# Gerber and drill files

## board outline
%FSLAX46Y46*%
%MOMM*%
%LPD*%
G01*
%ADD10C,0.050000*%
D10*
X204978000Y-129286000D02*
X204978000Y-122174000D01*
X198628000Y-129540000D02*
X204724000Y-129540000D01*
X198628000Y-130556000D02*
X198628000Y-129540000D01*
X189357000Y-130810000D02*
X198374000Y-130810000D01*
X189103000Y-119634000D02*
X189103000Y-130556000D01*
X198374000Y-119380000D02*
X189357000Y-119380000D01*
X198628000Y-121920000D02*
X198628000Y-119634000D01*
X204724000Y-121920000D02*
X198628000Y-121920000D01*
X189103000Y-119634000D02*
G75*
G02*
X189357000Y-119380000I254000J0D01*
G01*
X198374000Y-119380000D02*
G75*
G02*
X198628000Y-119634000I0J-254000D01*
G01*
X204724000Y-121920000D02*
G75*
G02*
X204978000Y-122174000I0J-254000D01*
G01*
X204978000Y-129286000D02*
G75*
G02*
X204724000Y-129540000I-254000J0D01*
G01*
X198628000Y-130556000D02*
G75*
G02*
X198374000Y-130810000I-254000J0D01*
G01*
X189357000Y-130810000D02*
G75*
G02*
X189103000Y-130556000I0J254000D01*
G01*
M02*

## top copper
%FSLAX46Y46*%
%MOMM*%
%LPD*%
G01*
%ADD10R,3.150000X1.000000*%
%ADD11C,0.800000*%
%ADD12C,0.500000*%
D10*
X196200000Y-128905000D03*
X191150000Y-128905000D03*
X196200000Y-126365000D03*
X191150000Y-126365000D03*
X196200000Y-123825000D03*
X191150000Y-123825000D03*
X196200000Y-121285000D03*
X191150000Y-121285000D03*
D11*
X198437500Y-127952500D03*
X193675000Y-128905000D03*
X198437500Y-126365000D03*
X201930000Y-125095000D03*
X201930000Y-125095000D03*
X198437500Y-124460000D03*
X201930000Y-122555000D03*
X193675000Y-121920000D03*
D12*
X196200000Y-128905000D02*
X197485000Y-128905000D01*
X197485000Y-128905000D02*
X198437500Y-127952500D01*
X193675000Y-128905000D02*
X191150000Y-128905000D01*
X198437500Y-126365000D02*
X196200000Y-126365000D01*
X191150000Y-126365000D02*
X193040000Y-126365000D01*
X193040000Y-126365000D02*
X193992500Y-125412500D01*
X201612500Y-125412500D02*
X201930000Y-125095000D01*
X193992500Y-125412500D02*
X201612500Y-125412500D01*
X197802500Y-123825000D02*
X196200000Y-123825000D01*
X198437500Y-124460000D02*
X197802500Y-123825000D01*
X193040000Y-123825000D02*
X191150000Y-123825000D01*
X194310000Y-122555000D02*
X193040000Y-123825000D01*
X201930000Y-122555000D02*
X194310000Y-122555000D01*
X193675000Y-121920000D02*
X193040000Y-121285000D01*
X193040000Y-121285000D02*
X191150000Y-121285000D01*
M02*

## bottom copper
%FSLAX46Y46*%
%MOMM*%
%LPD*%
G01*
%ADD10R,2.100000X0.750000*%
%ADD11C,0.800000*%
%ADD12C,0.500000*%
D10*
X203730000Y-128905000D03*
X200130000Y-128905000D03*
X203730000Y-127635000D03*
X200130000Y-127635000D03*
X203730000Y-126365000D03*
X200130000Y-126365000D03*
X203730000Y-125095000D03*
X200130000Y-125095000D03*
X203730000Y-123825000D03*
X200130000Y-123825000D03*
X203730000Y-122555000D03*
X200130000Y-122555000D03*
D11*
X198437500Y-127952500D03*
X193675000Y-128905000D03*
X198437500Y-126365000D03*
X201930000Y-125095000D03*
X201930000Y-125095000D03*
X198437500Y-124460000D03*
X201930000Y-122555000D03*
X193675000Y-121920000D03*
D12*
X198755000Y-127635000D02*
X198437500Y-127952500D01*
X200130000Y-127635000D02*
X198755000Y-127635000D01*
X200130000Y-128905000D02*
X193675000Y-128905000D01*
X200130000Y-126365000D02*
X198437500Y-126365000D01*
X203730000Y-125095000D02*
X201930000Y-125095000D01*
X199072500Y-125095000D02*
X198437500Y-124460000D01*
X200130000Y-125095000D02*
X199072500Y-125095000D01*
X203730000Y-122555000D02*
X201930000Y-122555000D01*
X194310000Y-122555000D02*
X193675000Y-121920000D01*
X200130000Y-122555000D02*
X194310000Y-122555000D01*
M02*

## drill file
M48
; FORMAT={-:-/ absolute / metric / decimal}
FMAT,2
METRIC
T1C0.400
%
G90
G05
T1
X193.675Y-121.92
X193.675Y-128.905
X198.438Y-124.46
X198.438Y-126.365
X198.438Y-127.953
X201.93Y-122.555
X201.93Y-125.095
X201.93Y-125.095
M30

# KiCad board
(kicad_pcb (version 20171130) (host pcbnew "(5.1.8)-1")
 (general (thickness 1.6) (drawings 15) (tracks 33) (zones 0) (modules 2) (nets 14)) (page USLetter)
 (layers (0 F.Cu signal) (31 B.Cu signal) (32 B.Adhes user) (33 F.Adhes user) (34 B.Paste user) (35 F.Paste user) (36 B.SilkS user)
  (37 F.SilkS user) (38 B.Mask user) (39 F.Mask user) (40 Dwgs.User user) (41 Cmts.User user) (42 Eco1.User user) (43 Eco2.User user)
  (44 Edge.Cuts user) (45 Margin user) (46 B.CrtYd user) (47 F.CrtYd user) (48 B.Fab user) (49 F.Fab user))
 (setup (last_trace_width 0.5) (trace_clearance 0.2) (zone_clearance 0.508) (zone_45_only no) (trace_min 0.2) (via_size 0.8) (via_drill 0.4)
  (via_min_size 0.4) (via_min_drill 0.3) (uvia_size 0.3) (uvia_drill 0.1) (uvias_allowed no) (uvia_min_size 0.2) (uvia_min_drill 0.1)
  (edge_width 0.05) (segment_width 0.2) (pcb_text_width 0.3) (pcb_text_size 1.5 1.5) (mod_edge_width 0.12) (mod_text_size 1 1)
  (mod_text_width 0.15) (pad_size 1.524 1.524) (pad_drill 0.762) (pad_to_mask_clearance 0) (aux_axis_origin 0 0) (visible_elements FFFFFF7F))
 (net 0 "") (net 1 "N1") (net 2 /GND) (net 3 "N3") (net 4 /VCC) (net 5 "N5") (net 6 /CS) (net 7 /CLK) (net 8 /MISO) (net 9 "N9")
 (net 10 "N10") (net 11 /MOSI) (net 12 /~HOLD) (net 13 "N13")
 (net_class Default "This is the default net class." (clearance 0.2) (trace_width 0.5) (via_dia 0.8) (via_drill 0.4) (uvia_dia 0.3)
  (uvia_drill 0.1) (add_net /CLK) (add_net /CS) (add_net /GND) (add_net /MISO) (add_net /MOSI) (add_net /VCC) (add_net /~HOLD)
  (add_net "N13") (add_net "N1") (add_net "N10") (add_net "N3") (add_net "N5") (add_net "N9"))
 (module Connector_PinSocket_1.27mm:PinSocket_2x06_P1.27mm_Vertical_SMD (layer B.Cu) (at 201.93 125.73)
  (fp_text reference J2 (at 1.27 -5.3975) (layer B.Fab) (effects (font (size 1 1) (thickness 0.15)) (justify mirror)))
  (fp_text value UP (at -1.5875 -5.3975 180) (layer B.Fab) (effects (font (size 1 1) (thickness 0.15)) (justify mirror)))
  (pad 1 smd rect (at 1.8 3.175) (size 2.1 0.75) (layers B.Cu B.Paste B.Mask) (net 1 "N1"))
  (pad 2 smd rect (at -1.8 3.175) (size 2.1 0.75) (layers B.Cu B.Paste B.Mask) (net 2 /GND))
  (pad 3 smd rect (at 1.8 1.905) (size 2.1 0.75) (layers B.Cu B.Paste B.Mask) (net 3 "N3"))
  (pad 4 smd rect (at -1.8 1.905) (size 2.1 0.75) (layers B.Cu B.Paste B.Mask) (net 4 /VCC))
  (pad 5 smd rect (at 1.8 0.635) (size 2.1 0.75) (layers B.Cu B.Paste B.Mask) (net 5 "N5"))
  (pad 6 smd rect (at -1.8 0.635) (size 2.1 0.75) (layers B.Cu B.Paste B.Mask) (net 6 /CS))
  (pad 7 smd rect (at 1.8 -0.635) (size 2.1 0.75) (layers B.Cu B.Paste B.Mask) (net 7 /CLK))
  (pad 8 smd rect (at -1.8 -0.635) (size 2.1 0.75) (layers B.Cu B.Paste B.Mask) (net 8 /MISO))
  (pad 9 smd rect (at 1.8 -1.905) (size 2.1 0.75) (layers B.Cu B.Paste B.Mask) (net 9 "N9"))
  (pad 10 smd rect (at -1.8 -1.905) (size 2.1 0.75) (layers B.Cu B.Paste B.Mask) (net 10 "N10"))
  (pad 11 smd rect (at 1.8 -3.175) (size 2.1 0.75) (layers B.Cu B.Paste B.Mask) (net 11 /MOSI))
  (pad 12 smd rect (at -1.8 -3.175) (size 2.1 0.75) (layers B.Cu B.Paste B.Mask) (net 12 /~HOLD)))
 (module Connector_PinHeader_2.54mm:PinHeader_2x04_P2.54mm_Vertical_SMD (layer F.Cu) (at 193.675 125.095 180)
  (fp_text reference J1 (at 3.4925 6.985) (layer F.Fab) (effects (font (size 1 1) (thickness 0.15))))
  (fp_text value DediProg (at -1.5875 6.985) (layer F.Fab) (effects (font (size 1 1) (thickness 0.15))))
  (pad 1 smd rect (at -2.525 -3.81 180) (size 3.15 1) (layers F.Cu F.Paste F.Mask) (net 4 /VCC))
  (pad 2 smd rect (at 2.525 -3.81 180) (size 3.15 1) (layers F.Cu F.Paste F.Mask) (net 2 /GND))
  (pad 3 smd rect (at -2.525 -1.27 180) (size 3.15 1) (layers F.Cu F.Paste F.Mask) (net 6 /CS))
  (pad 4 smd rect (at 2.525 -1.27 180) (size 3.15 1) (layers F.Cu F.Paste F.Mask) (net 7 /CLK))
  (pad 5 smd rect (at -2.525 1.27 180) (size 3.15 1) (layers F.Cu F.Paste F.Mask) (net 8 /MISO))
  (pad 6 smd rect (at 2.525 1.27 180) (size 3.15 1) (layers F.Cu F.Paste F.Mask) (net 11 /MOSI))
  (pad 7 smd rect (at -2.525 3.81 180) (size 3.15 1) (layers F.Cu F.Paste F.Mask) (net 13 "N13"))
  (pad 8 smd rect (at 2.525 3.81 180) (size 3.15 1) (layers F.Cu F.Paste F.Mask) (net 12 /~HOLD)))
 (gr_line (start 204.978 129.286) (end 204.978 122.174) (layer Edge.Cuts) (width 0.05))
 (gr_line (start 198.628 129.54) (end 204.724 129.54) (layer Edge.Cuts) (width 0.05))
 (gr_line (start 198.628 130.556) (end 198.628 129.54) (layer Edge.Cuts) (width 0.05))
 (gr_line (start 189.357 130.81) (end 198.374 130.81) (layer Edge.Cuts) (width 0.05))
 (gr_line (start 189.103 119.634) (end 189.103 130.556) (layer Edge.Cuts) (width 0.05))
 (gr_line (start 198.374 119.38) (end 189.357 119.38) (layer Edge.Cuts) (width 0.05))
 (gr_line (start 198.628 121.92) (end 198.628 119.634) (layer Edge.Cuts) (width 0.05))
 (gr_line (start 204.724 121.92) (end 198.628 121.92) (layer Edge.Cuts) (width 0.05))
 (gr_arc (start 189.357 119.634) (end 189.357 119.38) (angle -90) (layer Edge.Cuts) (width 0.05))
 (gr_arc (start 198.374 119.634) (end 198.628 119.634) (angle -90) (layer Edge.Cuts) (width 0.05))
 (gr_arc (start 204.724 122.174) (end 204.978 122.174) (angle -90) (layer Edge.Cuts) (width 0.05))
 (gr_arc (start 204.724 129.286) (end 204.724 129.54) (angle -90) (layer Edge.Cuts) (width 0.05))
 (gr_arc (start 198.374 130.556) (end 198.374 130.81) (angle -90) (layer Edge.Cuts) (width 0.05))
 (gr_arc (start 189.357 130.556) (end 189.103 130.556) (angle -90) (layer Edge.Cuts) (width 0.05))
 (via (at 198.4375 127.9525) (size 0.8) (drill 0.4) (layers F.Cu B.Cu) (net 4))
 (segment (start 196.2 128.905) (end 197.485 128.905) (width 0.5) (layer F.Cu) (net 4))
 (segment (start 197.485 128.905) (end 198.4375 127.9525) (width 0.5) (layer F.Cu) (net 4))
 (segment (start 198.755 127.635) (end 198.4375 127.9525) (width 0.5) (layer B.Cu) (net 4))
 (segment (start 200.13 127.635) (end 198.755 127.635) (width 0.5) (layer B.Cu) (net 4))
 (via (at 193.675 128.905) (size 0.8) (drill 0.4) (layers F.Cu B.Cu) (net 2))
 (segment (start 200.13 128.905) (end 193.675 128.905) (width 0.5) (layer B.Cu) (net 2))
 (segment (start 193.675 128.905) (end 191.15 128.905) (width 0.5) (layer F.Cu) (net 2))
 (via (at 198.4375 126.365) (size 0.8) (drill 0.4) (layers F.Cu B.Cu) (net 6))
 (segment (start 200.13 126.365) (end 198.4375 126.365) (width 0.5) (layer B.Cu) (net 6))
 (segment (start 198.4375 126.365) (end 196.2 126.365) (width 0.5) (layer F.Cu) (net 6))
 (via (at 201.93 125.095) (size 0.8) (drill 0.4) (layers F.Cu B.Cu) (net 7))
 (segment (start 203.73 125.095) (end 201.93 125.095) (width 0.5) (layer B.Cu) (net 7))
 (via (at 201.93 125.095) (size 0.8) (drill 0.4) (layers F.Cu B.Cu) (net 7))
 (segment (start 191.15 126.365) (end 193.04 126.365) (width 0.5) (layer F.Cu) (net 7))
 (segment (start 193.04 126.365) (end 193.9925 125.4125) (width 0.5) (layer F.Cu) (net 7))
 (segment (start 201.6125 125.4125) (end 201.93 125.095) (width 0.5) (layer F.Cu) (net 7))
 (segment (start 193.9925 125.4125) (end 201.6125 125.4125) (width 0.5) (layer F.Cu) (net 7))
 (via (at 198.4375 124.46) (size 0.8) (drill 0.4) (layers F.Cu B.Cu) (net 8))
 (segment (start 199.0725 125.095) (end 198.4375 124.46) (width 0.5) (layer B.Cu) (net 8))
 (segment (start 200.13 125.095) (end 199.0725 125.095) (width 0.5) (layer B.Cu) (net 8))
 (segment (start 197.8025 123.825) (end 196.2 123.825) (width 0.5) (layer F.Cu) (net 8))
 (segment (start 198.4375 124.46) (end 197.8025 123.825) (width 0.5) (layer F.Cu) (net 8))
 (via (at 201.93 122.555) (size 0.8) (drill 0.4) (layers F.Cu B.Cu) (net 11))
 (segment (start 203.73 122.555) (end 201.93 122.555) (width 0.5) (layer B.Cu) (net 11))
 (segment (start 193.04 123.825) (end 191.15 123.825) (width 0.5) (layer F.Cu) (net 11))
 (segment (start 194.31 122.555) (end 193.04 123.825) (width 0.5) (layer F.Cu) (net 11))
 (segment (start 201.93 122.555) (end 194.31 122.555) (width 0.5) (layer F.Cu) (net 11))
 (via (at 193.675 121.92) (size 0.8) (drill 0.4) (layers F.Cu B.Cu) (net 12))
 (segment (start 194.31 122.555) (end 193.675 121.92) (width 0.5) (layer B.Cu) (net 12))
 (segment (start 200.13 122.555) (end 194.31 122.555) (width 0.5) (layer B.Cu) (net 12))
 (segment (start 193.675 121.92) (end 193.04 121.285) (width 0.5) (layer F.Cu) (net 12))
 (segment (start 193.04 121.285) (end 191.15 121.285) (width 0.5) (layer F.Cu) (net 12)))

